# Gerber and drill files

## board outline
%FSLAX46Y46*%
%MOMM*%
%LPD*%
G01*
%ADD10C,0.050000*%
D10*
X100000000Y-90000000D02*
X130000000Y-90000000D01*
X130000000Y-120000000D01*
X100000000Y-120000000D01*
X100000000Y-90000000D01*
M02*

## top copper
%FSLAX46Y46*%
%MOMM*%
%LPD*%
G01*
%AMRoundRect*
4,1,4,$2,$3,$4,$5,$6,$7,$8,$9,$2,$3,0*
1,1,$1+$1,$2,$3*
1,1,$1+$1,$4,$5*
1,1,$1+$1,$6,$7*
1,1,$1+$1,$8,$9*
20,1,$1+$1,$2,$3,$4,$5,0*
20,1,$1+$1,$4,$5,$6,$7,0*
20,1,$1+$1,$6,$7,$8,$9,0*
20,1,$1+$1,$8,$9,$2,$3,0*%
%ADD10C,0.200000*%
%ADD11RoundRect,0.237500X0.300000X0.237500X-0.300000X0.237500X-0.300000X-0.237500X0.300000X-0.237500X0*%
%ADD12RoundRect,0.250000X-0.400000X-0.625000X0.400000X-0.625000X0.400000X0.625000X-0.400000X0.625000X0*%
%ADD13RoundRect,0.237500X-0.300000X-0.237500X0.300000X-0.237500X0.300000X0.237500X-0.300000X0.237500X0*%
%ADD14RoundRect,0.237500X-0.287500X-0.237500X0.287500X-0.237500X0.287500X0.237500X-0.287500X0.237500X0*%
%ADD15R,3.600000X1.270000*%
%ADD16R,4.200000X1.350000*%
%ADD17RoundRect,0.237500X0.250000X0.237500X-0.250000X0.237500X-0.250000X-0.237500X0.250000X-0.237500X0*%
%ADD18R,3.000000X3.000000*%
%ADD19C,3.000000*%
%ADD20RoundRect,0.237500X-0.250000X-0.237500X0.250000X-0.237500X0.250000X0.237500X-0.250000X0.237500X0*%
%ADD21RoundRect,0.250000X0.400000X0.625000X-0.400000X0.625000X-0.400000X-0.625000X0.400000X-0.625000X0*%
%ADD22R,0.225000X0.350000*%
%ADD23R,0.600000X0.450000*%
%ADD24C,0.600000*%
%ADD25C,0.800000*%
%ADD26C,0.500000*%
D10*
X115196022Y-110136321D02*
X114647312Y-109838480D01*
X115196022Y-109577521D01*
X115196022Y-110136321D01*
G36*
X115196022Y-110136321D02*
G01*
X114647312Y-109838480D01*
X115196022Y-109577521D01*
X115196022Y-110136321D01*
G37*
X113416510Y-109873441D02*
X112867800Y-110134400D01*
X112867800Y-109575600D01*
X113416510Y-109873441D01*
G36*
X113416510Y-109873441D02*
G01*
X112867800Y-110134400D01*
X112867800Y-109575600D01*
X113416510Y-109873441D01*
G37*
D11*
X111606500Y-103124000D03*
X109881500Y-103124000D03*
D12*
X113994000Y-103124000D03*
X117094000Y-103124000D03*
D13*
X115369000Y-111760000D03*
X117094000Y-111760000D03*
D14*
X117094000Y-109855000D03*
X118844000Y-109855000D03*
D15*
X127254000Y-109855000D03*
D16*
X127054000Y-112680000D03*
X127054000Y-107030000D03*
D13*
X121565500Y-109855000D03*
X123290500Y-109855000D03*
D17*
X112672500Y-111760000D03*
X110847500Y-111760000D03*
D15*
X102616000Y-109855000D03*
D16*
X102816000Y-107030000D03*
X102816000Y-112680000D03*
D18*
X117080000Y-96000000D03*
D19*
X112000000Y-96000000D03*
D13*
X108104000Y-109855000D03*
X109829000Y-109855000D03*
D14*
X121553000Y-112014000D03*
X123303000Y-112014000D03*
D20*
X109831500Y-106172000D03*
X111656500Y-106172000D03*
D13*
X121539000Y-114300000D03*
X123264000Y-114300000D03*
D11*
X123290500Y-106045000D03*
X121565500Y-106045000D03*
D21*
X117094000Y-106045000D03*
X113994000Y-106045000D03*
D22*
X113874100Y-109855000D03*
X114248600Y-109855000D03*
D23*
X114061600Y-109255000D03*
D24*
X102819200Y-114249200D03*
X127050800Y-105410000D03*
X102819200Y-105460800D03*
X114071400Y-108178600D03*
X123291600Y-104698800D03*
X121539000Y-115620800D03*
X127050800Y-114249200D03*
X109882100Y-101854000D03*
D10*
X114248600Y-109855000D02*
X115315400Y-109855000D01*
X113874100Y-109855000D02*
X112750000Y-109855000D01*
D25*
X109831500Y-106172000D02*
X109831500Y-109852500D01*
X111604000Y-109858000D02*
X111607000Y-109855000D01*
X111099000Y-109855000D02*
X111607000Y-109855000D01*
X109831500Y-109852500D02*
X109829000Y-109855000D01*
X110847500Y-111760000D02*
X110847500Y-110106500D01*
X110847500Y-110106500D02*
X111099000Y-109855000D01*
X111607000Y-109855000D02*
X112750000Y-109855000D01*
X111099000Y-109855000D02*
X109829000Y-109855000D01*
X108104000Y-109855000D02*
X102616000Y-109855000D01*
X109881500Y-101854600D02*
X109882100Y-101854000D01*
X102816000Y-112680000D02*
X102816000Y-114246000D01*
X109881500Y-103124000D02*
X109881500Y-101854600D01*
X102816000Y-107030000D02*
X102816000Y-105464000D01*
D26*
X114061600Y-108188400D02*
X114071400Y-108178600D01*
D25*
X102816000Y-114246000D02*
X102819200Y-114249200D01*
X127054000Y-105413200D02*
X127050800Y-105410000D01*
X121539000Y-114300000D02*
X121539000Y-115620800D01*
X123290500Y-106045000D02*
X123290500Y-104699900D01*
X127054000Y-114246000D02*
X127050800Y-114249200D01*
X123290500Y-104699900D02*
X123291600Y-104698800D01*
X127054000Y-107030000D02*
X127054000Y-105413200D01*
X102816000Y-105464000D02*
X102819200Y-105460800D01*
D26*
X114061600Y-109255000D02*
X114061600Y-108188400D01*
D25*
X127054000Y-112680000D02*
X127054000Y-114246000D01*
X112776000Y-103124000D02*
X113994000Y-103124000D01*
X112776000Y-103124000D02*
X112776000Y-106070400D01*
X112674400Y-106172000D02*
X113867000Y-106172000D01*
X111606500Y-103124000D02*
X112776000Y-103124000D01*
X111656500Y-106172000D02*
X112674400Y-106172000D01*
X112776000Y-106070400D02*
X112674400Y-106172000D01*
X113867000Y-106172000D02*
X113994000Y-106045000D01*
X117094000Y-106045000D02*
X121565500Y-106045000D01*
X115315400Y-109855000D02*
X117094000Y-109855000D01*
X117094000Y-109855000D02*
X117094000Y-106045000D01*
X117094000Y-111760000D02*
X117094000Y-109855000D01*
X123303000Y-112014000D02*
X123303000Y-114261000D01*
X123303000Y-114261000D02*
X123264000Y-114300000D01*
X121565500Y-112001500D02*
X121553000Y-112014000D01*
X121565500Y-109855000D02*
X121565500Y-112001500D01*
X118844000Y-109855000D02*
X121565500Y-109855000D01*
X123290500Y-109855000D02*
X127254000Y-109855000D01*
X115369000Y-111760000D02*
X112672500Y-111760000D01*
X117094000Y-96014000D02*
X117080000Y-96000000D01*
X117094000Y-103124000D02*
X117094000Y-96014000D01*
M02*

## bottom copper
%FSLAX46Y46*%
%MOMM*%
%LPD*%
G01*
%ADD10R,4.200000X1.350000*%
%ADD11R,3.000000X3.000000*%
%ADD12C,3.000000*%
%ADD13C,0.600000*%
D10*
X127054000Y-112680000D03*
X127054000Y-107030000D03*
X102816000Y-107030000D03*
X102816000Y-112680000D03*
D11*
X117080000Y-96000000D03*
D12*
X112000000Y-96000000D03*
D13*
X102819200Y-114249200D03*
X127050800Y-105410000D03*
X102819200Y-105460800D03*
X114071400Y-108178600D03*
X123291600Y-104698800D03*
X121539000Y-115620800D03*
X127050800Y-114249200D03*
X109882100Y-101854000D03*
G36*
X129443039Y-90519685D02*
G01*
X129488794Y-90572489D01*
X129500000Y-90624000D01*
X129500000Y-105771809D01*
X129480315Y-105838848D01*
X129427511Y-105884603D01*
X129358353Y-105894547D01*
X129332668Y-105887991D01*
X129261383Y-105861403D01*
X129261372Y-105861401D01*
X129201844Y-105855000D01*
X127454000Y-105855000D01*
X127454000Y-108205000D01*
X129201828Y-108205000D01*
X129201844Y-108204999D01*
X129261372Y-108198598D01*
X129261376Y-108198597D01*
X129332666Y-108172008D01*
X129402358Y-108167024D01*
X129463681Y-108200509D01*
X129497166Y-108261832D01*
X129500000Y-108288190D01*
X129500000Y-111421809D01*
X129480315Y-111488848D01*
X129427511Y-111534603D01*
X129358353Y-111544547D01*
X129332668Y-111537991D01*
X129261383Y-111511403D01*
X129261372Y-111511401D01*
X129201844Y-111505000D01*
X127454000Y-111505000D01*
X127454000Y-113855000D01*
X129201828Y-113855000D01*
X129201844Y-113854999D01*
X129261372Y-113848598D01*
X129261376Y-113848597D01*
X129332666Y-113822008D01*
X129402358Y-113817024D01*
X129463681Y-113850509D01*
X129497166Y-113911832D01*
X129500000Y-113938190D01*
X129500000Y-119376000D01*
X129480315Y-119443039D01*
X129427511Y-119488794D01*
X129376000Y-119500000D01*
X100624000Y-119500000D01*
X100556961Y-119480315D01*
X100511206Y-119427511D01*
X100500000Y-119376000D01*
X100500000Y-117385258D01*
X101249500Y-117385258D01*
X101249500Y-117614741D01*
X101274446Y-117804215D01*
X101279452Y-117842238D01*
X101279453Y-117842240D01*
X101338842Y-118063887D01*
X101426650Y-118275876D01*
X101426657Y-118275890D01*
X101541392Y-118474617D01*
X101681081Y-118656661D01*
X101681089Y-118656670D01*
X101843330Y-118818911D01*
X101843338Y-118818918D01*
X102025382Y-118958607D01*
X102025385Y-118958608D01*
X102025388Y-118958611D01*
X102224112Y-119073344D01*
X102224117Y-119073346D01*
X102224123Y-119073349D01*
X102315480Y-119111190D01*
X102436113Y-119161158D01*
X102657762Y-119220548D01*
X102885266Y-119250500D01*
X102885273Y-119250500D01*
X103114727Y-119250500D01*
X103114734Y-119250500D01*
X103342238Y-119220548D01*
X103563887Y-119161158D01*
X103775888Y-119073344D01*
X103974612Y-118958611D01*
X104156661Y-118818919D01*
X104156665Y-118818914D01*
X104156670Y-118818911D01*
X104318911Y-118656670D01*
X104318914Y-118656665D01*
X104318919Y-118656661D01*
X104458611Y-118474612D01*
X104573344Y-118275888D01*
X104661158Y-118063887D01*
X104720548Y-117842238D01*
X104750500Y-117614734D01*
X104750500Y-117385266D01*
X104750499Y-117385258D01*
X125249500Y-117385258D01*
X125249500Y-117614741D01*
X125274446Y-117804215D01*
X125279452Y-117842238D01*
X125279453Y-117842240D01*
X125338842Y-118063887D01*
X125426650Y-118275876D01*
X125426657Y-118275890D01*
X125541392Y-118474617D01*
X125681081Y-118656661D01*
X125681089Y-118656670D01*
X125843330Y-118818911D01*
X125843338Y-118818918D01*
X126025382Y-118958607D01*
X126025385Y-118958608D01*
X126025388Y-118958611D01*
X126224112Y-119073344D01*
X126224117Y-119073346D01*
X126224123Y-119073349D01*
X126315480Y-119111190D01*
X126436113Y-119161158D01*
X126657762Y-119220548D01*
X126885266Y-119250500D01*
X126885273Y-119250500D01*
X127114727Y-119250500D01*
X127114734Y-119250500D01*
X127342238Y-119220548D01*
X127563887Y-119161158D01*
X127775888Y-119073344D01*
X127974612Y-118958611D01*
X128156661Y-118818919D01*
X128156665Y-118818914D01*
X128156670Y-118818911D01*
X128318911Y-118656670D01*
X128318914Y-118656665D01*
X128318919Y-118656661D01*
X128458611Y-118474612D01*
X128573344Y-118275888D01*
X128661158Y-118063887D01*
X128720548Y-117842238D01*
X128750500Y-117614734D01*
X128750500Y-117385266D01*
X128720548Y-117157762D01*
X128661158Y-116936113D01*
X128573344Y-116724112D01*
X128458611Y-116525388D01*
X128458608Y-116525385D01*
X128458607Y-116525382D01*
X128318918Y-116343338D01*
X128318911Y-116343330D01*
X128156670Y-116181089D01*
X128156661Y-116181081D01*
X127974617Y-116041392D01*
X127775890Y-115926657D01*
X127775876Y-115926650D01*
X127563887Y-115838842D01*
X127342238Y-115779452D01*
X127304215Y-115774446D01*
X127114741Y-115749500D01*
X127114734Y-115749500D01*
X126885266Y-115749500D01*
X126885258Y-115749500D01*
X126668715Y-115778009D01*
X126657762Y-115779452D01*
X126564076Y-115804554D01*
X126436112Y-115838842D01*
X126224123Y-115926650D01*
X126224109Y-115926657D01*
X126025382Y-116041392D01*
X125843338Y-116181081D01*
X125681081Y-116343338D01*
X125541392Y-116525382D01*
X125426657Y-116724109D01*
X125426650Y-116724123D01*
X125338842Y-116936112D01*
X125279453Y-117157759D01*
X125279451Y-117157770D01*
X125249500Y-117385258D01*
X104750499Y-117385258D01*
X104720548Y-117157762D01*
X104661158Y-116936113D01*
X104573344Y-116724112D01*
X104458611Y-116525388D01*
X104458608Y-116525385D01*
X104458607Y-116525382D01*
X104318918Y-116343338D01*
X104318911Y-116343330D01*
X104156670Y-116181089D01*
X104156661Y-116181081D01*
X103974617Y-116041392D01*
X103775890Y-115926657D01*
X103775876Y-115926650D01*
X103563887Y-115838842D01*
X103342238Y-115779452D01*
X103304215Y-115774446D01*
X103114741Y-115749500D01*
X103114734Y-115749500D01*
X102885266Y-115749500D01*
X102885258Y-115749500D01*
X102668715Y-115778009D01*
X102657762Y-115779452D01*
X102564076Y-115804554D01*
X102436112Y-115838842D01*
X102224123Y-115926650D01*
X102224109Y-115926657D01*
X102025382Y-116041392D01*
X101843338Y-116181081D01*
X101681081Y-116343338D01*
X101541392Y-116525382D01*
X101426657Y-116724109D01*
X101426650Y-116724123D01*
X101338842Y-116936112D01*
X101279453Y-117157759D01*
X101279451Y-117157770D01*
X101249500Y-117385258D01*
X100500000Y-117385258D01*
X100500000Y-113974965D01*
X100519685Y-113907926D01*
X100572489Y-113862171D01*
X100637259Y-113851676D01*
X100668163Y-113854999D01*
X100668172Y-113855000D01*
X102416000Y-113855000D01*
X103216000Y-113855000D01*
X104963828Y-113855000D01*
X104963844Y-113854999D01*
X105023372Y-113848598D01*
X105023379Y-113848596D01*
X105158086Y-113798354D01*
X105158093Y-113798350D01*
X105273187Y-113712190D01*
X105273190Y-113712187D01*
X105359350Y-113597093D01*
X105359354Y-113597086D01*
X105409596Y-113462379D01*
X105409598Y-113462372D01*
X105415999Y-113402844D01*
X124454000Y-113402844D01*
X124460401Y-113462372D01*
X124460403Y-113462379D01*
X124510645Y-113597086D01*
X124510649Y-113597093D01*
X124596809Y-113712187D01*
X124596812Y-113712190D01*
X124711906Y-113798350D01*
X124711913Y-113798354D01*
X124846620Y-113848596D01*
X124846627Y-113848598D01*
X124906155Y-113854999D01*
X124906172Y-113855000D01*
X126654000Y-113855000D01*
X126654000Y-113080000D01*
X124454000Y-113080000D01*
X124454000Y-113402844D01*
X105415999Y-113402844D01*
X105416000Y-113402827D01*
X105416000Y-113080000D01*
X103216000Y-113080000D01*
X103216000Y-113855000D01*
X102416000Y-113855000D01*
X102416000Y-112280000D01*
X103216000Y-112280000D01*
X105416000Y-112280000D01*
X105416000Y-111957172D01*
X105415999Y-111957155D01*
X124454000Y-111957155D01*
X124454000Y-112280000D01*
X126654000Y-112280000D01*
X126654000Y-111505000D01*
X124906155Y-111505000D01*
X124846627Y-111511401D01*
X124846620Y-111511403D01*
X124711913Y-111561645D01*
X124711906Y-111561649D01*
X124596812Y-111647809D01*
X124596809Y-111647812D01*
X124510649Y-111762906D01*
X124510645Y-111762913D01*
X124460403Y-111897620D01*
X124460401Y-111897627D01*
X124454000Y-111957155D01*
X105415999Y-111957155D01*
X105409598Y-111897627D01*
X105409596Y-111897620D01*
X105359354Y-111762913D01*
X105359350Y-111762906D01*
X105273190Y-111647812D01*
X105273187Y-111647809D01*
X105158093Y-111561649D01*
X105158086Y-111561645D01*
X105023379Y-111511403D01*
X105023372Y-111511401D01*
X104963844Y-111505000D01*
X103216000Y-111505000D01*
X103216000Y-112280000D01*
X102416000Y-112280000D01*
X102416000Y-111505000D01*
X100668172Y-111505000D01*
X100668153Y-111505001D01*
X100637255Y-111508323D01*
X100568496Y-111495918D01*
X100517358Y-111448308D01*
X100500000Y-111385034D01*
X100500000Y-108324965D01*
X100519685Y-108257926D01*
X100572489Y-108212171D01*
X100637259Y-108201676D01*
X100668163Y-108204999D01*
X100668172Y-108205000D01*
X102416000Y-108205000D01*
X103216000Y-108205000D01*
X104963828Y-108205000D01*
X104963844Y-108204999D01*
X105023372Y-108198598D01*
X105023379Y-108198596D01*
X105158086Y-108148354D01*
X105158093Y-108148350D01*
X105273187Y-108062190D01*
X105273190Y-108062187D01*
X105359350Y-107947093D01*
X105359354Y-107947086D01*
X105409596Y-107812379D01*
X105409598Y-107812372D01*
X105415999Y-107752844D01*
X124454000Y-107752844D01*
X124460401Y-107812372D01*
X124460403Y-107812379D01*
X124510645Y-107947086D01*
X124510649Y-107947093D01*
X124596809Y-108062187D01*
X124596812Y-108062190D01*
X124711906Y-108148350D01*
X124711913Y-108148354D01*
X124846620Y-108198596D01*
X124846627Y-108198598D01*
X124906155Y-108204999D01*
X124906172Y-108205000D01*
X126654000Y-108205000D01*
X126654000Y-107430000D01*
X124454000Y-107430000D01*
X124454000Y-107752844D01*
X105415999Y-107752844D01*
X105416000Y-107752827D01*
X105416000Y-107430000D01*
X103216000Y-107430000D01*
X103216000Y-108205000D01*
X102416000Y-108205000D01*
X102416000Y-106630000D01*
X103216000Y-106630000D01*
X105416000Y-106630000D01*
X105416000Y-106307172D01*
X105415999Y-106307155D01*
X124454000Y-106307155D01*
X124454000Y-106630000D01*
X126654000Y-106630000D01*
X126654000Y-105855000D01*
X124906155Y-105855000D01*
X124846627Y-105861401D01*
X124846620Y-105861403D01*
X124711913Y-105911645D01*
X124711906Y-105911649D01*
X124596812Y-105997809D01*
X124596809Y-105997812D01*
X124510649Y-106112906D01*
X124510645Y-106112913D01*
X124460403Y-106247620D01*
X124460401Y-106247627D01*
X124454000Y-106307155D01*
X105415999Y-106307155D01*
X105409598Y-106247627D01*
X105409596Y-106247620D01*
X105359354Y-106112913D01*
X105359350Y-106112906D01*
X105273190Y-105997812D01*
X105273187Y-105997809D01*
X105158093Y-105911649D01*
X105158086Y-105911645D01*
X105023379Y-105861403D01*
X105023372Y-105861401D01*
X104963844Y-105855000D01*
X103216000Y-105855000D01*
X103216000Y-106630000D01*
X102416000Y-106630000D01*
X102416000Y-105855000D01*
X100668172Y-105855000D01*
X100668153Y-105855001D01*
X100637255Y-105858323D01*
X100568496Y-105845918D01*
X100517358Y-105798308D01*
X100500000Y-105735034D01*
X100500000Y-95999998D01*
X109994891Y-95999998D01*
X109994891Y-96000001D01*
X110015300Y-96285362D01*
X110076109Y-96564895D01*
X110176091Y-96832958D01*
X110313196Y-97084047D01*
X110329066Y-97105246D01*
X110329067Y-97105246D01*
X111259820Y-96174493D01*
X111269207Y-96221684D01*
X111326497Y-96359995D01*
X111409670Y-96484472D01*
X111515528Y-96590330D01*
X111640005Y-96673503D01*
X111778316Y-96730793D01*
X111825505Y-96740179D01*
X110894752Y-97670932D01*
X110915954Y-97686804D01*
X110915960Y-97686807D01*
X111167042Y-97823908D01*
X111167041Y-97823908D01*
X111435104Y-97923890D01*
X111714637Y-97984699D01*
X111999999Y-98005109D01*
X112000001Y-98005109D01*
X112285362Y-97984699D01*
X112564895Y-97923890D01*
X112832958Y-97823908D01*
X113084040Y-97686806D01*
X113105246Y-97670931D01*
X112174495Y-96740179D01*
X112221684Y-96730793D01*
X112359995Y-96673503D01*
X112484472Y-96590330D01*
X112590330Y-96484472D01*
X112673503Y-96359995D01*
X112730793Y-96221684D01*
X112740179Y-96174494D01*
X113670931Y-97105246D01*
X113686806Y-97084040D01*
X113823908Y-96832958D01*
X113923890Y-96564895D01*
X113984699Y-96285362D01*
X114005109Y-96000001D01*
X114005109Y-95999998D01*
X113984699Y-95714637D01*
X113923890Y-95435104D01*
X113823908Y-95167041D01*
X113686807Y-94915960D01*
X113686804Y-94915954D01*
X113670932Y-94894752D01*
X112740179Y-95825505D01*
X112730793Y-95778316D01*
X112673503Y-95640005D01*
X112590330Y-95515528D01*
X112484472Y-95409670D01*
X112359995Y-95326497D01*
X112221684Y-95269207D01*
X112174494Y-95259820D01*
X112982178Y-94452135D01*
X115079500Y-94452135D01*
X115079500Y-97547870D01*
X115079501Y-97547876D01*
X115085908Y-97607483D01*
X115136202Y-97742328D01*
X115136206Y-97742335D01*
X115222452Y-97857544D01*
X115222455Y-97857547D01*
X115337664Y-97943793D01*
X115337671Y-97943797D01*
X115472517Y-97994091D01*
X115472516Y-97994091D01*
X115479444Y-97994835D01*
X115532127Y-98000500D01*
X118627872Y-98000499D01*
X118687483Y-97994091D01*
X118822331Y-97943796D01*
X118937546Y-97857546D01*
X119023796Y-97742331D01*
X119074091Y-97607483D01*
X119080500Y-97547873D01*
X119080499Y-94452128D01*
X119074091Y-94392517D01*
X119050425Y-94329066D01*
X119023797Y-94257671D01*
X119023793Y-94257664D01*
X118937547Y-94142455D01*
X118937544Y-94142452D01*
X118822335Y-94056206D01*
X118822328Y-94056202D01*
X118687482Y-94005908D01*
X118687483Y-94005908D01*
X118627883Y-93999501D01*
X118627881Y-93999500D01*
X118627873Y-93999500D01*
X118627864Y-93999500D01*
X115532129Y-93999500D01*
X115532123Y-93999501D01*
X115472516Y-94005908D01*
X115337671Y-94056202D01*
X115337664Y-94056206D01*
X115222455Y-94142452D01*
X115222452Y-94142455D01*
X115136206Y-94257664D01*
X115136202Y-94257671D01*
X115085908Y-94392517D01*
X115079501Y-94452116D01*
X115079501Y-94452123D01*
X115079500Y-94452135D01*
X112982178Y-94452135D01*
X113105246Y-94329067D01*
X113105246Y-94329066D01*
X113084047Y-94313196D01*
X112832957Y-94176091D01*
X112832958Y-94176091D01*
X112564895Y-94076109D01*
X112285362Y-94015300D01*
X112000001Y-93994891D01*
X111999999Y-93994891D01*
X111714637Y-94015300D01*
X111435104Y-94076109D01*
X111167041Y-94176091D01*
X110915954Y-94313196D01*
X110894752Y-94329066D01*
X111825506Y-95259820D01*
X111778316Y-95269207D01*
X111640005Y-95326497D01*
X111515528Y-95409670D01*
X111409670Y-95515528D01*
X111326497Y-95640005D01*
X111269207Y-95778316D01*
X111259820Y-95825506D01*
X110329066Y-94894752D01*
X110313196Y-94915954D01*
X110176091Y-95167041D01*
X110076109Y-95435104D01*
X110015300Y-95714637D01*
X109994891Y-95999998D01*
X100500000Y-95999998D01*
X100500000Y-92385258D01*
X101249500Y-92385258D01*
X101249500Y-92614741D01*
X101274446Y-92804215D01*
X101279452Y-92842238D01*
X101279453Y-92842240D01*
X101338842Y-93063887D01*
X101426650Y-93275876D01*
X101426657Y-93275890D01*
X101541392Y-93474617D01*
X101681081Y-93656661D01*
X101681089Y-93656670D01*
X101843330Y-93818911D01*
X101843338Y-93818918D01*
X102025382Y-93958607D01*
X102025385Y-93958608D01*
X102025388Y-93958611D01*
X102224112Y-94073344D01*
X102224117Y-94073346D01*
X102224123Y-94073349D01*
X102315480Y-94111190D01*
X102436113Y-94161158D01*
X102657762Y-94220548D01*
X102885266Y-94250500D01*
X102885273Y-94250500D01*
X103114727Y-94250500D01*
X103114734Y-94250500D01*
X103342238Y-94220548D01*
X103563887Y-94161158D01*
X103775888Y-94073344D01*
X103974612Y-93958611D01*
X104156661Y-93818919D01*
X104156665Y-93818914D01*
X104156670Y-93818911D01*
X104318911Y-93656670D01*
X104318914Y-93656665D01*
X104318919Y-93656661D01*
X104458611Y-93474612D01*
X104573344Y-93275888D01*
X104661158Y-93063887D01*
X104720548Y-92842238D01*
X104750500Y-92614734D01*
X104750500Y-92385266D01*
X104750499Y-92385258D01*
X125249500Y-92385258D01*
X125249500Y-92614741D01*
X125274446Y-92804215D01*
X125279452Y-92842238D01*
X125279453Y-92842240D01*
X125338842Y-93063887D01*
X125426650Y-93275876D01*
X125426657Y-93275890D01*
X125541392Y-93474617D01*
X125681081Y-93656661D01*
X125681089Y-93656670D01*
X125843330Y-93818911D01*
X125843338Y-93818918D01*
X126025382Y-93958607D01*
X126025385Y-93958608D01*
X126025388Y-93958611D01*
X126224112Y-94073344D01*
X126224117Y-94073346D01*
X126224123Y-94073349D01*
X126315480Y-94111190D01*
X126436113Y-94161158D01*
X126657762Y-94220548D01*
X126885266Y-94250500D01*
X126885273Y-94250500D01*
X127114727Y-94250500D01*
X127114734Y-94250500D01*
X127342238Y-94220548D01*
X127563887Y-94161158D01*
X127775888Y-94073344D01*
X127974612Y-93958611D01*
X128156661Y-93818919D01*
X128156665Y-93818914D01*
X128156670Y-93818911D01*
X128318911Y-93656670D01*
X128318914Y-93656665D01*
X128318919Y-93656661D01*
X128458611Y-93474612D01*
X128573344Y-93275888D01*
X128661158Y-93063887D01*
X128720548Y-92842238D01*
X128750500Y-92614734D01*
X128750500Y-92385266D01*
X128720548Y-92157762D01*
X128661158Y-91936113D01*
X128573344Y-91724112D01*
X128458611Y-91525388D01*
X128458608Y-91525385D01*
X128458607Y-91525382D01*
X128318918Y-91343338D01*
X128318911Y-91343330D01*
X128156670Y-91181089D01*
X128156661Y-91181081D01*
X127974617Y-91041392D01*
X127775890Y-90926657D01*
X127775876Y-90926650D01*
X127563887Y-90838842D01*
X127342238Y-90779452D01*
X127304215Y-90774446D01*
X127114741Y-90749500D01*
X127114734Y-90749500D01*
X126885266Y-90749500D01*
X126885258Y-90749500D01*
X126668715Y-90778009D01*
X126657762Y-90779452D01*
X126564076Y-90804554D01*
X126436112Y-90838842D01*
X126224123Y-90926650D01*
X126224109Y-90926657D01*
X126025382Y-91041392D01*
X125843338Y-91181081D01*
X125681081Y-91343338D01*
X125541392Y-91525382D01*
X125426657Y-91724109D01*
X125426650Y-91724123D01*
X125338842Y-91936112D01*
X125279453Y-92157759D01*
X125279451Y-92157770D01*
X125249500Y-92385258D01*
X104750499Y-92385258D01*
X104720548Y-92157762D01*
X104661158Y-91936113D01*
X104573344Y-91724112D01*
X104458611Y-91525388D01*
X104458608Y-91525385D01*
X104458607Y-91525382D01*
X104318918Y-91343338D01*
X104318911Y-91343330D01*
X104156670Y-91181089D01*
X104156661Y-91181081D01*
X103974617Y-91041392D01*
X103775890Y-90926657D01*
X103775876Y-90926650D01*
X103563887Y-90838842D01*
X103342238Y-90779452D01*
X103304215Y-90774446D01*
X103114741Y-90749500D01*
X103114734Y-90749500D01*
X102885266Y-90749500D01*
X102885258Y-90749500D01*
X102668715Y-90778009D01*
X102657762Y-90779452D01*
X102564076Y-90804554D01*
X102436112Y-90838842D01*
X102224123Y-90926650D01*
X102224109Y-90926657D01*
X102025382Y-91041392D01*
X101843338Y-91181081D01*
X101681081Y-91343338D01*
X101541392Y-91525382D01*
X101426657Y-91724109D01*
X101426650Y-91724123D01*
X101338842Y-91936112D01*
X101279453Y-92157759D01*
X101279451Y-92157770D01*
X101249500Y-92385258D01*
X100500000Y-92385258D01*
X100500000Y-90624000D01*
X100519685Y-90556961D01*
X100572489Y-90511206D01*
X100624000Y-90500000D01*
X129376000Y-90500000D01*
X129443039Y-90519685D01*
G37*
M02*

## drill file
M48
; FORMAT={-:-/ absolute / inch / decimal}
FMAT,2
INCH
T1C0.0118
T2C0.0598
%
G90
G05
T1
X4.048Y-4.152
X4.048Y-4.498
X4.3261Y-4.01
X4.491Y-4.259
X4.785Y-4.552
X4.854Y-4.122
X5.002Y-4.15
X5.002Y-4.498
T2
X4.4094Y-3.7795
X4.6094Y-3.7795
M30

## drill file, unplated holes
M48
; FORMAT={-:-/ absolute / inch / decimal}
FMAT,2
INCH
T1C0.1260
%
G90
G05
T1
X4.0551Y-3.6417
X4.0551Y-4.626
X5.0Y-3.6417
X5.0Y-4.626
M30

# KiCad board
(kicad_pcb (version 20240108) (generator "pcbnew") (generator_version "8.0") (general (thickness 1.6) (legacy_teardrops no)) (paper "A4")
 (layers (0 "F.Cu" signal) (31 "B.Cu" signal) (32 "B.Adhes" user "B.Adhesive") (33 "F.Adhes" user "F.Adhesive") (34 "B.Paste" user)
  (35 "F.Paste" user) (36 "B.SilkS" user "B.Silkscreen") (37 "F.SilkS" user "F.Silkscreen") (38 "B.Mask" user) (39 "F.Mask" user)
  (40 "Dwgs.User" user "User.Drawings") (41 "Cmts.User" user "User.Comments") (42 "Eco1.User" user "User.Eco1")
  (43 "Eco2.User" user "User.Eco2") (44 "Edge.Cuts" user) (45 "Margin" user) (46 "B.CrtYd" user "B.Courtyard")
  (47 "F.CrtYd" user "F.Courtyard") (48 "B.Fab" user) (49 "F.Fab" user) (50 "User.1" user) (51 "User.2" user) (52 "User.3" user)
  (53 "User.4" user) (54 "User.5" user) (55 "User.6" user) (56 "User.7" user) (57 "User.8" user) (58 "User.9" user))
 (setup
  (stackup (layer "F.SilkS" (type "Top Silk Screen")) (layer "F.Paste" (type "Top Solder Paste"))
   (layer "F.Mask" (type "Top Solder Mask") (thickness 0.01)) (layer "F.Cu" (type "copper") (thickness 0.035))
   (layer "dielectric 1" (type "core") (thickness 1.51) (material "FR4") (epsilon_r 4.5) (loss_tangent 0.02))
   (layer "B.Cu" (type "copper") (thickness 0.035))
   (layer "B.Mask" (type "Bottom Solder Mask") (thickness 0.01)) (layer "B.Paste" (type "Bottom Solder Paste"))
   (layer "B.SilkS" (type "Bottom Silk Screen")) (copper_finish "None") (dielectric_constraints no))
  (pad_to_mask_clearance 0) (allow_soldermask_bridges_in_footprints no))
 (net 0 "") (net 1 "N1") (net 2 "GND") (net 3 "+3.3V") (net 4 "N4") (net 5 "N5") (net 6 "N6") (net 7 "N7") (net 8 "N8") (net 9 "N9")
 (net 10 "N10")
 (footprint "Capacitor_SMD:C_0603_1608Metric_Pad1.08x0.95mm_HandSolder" (layer "F.Cu") (at 110.744 103.124 180)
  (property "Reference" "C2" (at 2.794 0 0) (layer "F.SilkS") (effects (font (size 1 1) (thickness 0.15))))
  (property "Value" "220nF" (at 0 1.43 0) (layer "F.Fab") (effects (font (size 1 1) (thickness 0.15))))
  (pad "1" smd roundrect (at -0.8625 0 180) (size 1.075 0.95) (layers "F.Cu" "F.Paste" "F.Mask") (roundrect_rratio 0.25) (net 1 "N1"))
  (pad "2" smd roundrect (at 0.8625 0 180) (size 1.075 0.95) (layers "F.Cu" "F.Paste" "F.Mask") (roundrect_rratio 0.25) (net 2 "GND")))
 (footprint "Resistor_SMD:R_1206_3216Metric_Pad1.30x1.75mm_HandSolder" (layer "F.Cu") (at 115.544 103.124)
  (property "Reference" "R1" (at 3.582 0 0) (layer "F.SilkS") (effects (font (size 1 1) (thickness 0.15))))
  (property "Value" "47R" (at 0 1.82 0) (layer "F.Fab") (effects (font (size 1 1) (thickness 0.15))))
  (pad "1" smd roundrect (at -1.55 0) (size 1.3 1.75) (layers "F.Cu" "F.Paste" "F.Mask") (roundrect_rratio 0.192308) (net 1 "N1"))
  (pad "2" smd roundrect (at 1.55 0) (size 1.3 1.75) (layers "F.Cu" "F.Paste" "F.Mask") (roundrect_rratio 0.192308) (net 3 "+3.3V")))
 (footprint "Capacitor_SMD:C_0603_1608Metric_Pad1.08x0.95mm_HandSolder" (layer "F.Cu") (at 116.2315 111.76)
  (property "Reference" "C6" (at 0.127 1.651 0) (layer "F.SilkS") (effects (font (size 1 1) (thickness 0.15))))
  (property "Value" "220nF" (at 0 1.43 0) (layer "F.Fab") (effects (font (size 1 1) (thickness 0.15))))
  (pad "1" smd roundrect (at -0.8625 0) (size 1.075 0.95) (layers "F.Cu" "F.Paste" "F.Mask") (roundrect_rratio 0.25) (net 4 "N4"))
  (pad "2" smd roundrect (at 0.8625 0) (size 1.075 0.95) (layers "F.Cu" "F.Paste" "F.Mask") (roundrect_rratio 0.25) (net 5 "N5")))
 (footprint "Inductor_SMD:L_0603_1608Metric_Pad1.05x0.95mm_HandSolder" (layer "F.Cu") (at 117.969 109.855)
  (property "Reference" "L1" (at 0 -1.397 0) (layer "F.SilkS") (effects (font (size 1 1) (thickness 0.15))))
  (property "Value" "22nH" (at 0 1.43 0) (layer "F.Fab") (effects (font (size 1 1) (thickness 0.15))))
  (pad "1" smd roundrect (at -0.875 0) (size 1.05 0.95) (layers "F.Cu" "F.Paste" "F.Mask") (roundrect_rratio 0.25) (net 5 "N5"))
  (pad "2" smd roundrect (at 0.875 0) (size 1.05 0.95) (layers "F.Cu" "F.Paste" "F.Mask") (roundrect_rratio 0.25) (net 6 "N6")))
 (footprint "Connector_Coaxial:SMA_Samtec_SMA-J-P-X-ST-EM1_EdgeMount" (layer "F.Cu") (at 127.054 109.855 90)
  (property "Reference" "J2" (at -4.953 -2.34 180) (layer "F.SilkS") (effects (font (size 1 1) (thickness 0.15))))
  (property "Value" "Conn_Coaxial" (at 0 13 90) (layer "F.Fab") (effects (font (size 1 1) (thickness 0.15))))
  (pad "1" smd rect (at 0 0.2 90) (size 1.27 3.6) (layers "F.Cu" "F.Paste" "F.Mask") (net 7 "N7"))
  (pad "2" smd rect (at -2.825 0 90) (size 1.35 4.2) (layers "F.Cu" "F.Paste" "F.Mask") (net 2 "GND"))
  (pad "2" smd rect (at -2.825 0 90) (size 1.35 4.2) (layers "B.Cu" "B.Paste" "B.Mask") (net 2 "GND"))
  (pad "2" smd rect (at 2.825 0 90) (size 1.35 4.2) (layers "F.Cu" "F.Paste" "F.Mask") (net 2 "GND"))
  (pad "2" smd rect (at 2.825 0 90) (size 1.35 4.2) (layers "B.Cu" "B.Paste" "B.Mask") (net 2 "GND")))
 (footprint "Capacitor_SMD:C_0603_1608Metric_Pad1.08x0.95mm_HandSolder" (layer "F.Cu") (at 122.428 109.855)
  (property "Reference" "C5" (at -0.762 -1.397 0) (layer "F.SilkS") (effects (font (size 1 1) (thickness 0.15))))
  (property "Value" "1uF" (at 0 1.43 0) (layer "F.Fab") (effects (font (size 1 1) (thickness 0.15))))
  (pad "1" smd roundrect (at -0.8625 0) (size 1.075 0.95) (layers "F.Cu" "F.Paste" "F.Mask") (roundrect_rratio 0.25) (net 6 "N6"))
  (pad "2" smd roundrect (at 0.8625 0) (size 1.075 0.95) (layers "F.Cu" "F.Paste" "F.Mask") (roundrect_rratio 0.25) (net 7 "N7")))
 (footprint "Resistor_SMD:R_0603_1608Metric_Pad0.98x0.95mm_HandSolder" (layer "F.Cu") (at 111.76 111.76 180)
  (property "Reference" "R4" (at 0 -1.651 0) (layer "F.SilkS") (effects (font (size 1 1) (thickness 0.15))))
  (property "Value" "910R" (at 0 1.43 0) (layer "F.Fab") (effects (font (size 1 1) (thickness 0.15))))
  (pad "1" smd roundrect (at -0.9125 0 180) (size 0.975 0.95) (layers "F.Cu" "F.Paste" "F.Mask") (roundrect_rratio 0.25) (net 4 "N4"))
  (pad "2" smd roundrect (at 0.9125 0 180) (size 0.975 0.95) (layers "F.Cu" "F.Paste" "F.Mask") (roundrect_rratio 0.25) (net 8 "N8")))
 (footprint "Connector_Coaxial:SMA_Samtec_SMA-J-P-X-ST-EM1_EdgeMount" (layer "F.Cu") (at 102.816 109.855 -90)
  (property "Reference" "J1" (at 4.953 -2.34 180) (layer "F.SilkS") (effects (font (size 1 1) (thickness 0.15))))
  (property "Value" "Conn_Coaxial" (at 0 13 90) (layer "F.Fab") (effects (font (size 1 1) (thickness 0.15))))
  (pad "1" smd rect (at 0 0.2 270) (size 1.27 3.6) (layers "F.Cu" "F.Paste" "F.Mask") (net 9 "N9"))
  (pad "2" smd rect (at -2.825 0 270) (size 1.35 4.2) (layers "F.Cu" "F.Paste" "F.Mask") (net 2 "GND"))
  (pad "2" smd rect (at -2.825 0 270) (size 1.35 4.2) (layers "B.Cu" "B.Paste" "B.Mask") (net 2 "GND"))
  (pad "2" smd rect (at 2.825 0 270) (size 1.35 4.2) (layers "F.Cu" "F.Paste" "F.Mask") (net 2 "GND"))
  (pad "2" smd rect (at 2.825 0 270) (size 1.35 4.2) (layers "B.Cu" "B.Paste" "B.Mask") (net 2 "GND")))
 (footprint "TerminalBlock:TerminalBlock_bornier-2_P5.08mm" (layer "F.Cu") (at 117.08 96 180)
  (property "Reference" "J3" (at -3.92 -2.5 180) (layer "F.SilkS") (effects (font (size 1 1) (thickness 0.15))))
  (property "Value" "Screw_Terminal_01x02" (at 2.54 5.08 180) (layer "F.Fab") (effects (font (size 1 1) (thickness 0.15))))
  (pad "1" thru_hole rect (at 0 0 180) (size 3 3) (drill 1.52) (layers "*.Cu" "*.Mask") (remove_unused_layers no) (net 3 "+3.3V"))
  (pad "2" thru_hole circle (at 5.08 0 180) (size 3 3) (drill 1.52) (layers "*.Cu" "*.Mask") (remove_unused_layers no) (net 2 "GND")))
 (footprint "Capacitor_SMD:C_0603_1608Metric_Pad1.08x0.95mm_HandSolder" (layer "F.Cu") (at 108.9665 109.855)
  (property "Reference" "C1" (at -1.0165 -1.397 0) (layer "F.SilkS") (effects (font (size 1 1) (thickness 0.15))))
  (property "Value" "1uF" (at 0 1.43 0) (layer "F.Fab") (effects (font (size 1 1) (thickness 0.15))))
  (pad "1" smd roundrect (at -0.8625 0) (size 1.075 0.95) (layers "F.Cu" "F.Paste" "F.Mask") (roundrect_rratio 0.25) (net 9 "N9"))
  (pad "2" smd roundrect (at 0.8625 0) (size 1.075 0.95) (layers "F.Cu" "F.Paste" "F.Mask") (roundrect_rratio 0.25) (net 8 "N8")))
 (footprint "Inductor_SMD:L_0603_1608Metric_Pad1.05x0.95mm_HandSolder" (layer "F.Cu") (at 122.428 112.014)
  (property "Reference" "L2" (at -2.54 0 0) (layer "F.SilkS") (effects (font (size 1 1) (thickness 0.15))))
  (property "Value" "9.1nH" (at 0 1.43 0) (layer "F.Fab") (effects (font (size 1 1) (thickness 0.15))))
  (pad "1" smd roundrect (at -0.875 0) (size 1.05 0.95) (layers "F.Cu" "F.Paste" "F.Mask") (roundrect_rratio 0.25) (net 6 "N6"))
  (pad "2" smd roundrect (at 0.875 0) (size 1.05 0.95) (layers "F.Cu" "F.Paste" "F.Mask") (roundrect_rratio 0.25) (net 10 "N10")))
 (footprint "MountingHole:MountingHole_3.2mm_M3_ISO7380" (layer "F.Cu") (at 103 92.5)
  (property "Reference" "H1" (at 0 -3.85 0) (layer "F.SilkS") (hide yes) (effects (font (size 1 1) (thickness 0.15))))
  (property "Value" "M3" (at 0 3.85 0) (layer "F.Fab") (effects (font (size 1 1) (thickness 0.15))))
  (pad "" np_thru_hole circle (at 0 0) (size 3.2 3.2) (drill 3.2) (layers "*.Cu" "*.Mask")))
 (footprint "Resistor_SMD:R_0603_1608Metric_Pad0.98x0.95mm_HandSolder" (layer "F.Cu") (at 110.744 106.172)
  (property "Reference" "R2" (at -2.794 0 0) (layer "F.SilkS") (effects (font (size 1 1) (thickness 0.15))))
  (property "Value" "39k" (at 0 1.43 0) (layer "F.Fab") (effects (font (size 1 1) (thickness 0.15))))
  (pad "1" smd roundrect (at -0.9125 0) (size 0.975 0.95) (layers "F.Cu" "F.Paste" "F.Mask") (roundrect_rratio 0.25) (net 8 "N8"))
  (pad "2" smd roundrect (at 0.9125 0) (size 0.975 0.95) (layers "F.Cu" "F.Paste" "F.Mask") (roundrect_rratio 0.25) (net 1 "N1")))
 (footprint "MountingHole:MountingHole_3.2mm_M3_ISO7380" (layer "F.Cu") (at 127 92.5)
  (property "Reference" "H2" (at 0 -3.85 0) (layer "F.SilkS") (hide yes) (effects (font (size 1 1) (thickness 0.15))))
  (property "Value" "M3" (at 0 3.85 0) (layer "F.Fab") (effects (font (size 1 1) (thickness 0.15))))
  (pad "" np_thru_hole circle (at 0 0) (size 3.2 3.2) (drill 3.2) (layers "*.Cu" "*.Mask")))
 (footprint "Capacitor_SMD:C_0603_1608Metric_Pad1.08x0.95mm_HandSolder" (layer "F.Cu") (at 122.4015 114.3)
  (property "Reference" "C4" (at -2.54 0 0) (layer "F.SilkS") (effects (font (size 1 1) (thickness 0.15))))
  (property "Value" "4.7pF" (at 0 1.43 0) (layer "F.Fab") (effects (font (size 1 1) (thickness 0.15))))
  (pad "1" smd roundrect (at -0.8625 0) (size 1.075 0.95) (layers "F.Cu" "F.Paste" "F.Mask") (roundrect_rratio 0.25) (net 2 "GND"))
  (pad "2" smd roundrect (at 0.8625 0) (size 1.075 0.95) (layers "F.Cu" "F.Paste" "F.Mask") (roundrect_rratio 0.25) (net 10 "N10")))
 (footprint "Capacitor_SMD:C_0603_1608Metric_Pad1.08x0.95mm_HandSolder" (layer "F.Cu") (at 122.428 106.045 180)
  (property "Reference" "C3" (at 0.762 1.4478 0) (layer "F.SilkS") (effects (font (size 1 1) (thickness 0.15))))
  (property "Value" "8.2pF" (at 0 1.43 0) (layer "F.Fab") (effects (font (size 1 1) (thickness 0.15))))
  (pad "1" smd roundrect (at -0.8625 0 180) (size 1.075 0.95) (layers "F.Cu" "F.Paste" "F.Mask") (roundrect_rratio 0.25) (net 2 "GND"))
  (pad "2" smd roundrect (at 0.8625 0 180) (size 1.075 0.95) (layers "F.Cu" "F.Paste" "F.Mask") (roundrect_rratio 0.25) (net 5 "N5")))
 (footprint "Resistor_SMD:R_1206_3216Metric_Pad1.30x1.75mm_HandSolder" (layer "F.Cu") (at 115.544 106.045 180)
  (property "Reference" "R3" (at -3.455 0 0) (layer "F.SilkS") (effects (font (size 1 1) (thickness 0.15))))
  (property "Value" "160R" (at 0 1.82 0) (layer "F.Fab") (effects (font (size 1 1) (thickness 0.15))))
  (pad "1" smd roundrect (at -1.55 0 180) (size 1.3 1.75) (layers "F.Cu" "F.Paste" "F.Mask") (roundrect_rratio 0.192308) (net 5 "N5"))
  (pad "2" smd roundrect (at 1.55 0 180) (size 1.3 1.75) (layers "F.Cu" "F.Paste" "F.Mask") (roundrect_rratio 0.192308) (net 1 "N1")))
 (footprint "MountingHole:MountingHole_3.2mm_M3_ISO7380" (layer "F.Cu") (at 127 117.5)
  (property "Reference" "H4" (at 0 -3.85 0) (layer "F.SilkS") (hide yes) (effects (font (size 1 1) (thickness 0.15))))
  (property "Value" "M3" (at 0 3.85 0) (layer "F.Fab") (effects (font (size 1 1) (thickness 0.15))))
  (pad "" np_thru_hole circle (at 0 0) (size 3.2 3.2) (drill 3.2) (layers "*.Cu" "*.Mask")))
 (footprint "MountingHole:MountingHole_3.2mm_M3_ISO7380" (layer "F.Cu") (at 103 117.5)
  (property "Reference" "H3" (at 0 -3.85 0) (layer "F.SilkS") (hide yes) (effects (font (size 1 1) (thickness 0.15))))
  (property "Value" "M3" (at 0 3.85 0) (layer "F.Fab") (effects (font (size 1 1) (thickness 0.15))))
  (pad "" np_thru_hole circle (at 0 0) (size 3.2 3.2) (drill 3.2) (layers "*.Cu" "*.Mask")))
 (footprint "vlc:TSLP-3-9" (layer "F.Cu") (at 114.06135 109.555 90)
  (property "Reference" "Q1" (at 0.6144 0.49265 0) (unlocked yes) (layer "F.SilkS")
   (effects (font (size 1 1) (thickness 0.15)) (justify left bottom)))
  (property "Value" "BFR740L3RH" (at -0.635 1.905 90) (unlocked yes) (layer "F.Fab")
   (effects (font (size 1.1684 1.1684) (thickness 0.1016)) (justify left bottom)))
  (pad "1" smd rect (at -0.3 -0.18725 90) (size 0.35 0.225) (layers "F.Cu" "F.Paste") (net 8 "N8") (solder_mask_margin 0.1016)
   (clearance 0.15) (thermal_bridge_angle 0))
  (pad "2" smd rect (at -0.3 0.18725 90) (size 0.35 0.225) (layers "F.Cu" "F.Paste") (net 5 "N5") (solder_mask_margin 0.1016)
   (clearance 0.15) (thermal_bridge_angle 0))
  (pad "3" smd rect (at 0.3 0.00025 90) (size 0.45 0.6) (layers "F.Cu" "F.Paste") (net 2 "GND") (solder_mask_margin 0.1016)
   (thermal_bridge_angle 0)))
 (gr_poly
  (pts (xy 115.196022 109.577521) (xy 114.647312 109.83848) (xy 115.196022 110.136321)) (stroke (width 0.2) (type solid)) (fill solid)
  (layer "F.Cu") (net 5))
 (gr_poly
  (pts (xy 112.8678 110.1344) (xy 113.41651 109.873441) (xy 112.8678 109.5756)) (stroke (width 0.2) (type solid)) (fill solid)
  (layer "F.Cu") (net 8))
 (gr_rect (start 100 90) (end 130 120) (stroke (width 0.05) (type default)) (fill none) (layer "Edge.Cuts"))
 (segment (start 109.8315 106.172) (end 109.8315 109.8525) (width 0.8) (layer "F.Cu") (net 8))
 (segment (start 111.604 109.858) (end 111.607 109.855) (width 0.8) (layer "F.Cu") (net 8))
 (segment (start 111.099 109.855) (end 111.607 109.855) (width 0.8) (layer "F.Cu") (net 8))
 (segment (start 109.8315 109.8525) (end 109.829 109.855) (width 0.8) (layer "F.Cu") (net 8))
 (segment (start 110.8475 111.76) (end 110.8475 110.1065) (width 0.8) (layer "F.Cu") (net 8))
 (segment (start 110.8475 110.1065) (end 111.099 109.855) (width 0.8) (layer "F.Cu") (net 8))
 (segment (start 111.607 109.855) (end 112.75 109.855) (width 0.8) (layer "F.Cu") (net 8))
 (segment (start 113.8741 109.855) (end 112.75 109.855) (width 0.2) (layer "F.Cu") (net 8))
 (segment (start 111.099 109.855) (end 109.829 109.855) (width 0.8) (layer "F.Cu") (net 8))
 (segment (start 108.104 109.855) (end 102.616 109.855) (width 0.8) (layer "F.Cu") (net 9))
 (segment (start 109.8815 101.8546) (end 109.8821 101.854) (width 0.8) (layer "F.Cu") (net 2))
 (segment (start 102.816 112.68) (end 102.816 114.246) (width 0.8) (layer "F.Cu") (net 2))
 (segment (start 109.8815 103.124) (end 109.8815 101.8546) (width 0.8) (layer "F.Cu") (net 2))
 (segment (start 102.816 107.03) (end 102.816 105.464) (width 0.8) (layer "F.Cu") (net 2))
 (segment (start 114.0616 108.1884) (end 114.0714 108.1786) (width 0.5) (layer "F.Cu") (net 2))
 (segment (start 102.816 114.246) (end 102.8192 114.2492) (width 0.8) (layer "F.Cu") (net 2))
 (segment (start 127.054 105.4132) (end 127.0508 105.41) (width 0.8) (layer "F.Cu") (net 2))
 (segment (start 121.539 114.3) (end 121.539 115.6208) (width 0.8) (layer "F.Cu") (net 2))
 (segment (start 123.2905 106.045) (end 123.2905 104.6999) (width 0.8) (layer "F.Cu") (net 2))
 (segment (start 127.054 114.246) (end 127.0508 114.2492) (width 0.8) (layer "F.Cu") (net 2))
 (segment (start 123.2905 104.6999) (end 123.2916 104.6988) (width 0.8) (layer "F.Cu") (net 2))
 (segment (start 127.054 107.03) (end 127.054 105.4132) (width 0.8) (layer "F.Cu") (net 2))
 (segment (start 102.816 105.464) (end 102.8192 105.4608) (width 0.8) (layer "F.Cu") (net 2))
 (segment (start 114.0616 109.255) (end 114.0616 108.1884) (width 0.5) (layer "F.Cu") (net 2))
 (segment (start 127.054 112.68) (end 127.054 114.246) (width 0.8) (layer "F.Cu") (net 2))
 (via (at 102.8192 114.2492) (size 0.6) (drill 0.3) (layers "F.Cu" "B.Cu") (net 2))
 (via (at 127.0508 105.41) (size 0.6) (drill 0.3) (layers "F.Cu" "B.Cu") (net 2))
 (via (at 102.8192 105.4608) (size 0.6) (drill 0.3) (layers "F.Cu" "B.Cu") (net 2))
 (via (at 114.0714 108.1786) (size 0.6) (drill 0.3) (layers "F.Cu" "B.Cu") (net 2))
 (via (at 123.2916 104.6988) (size 0.6) (drill 0.3) (layers "F.Cu" "B.Cu") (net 2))
 (via (at 121.539 115.6208) (size 0.6) (drill 0.3) (layers "F.Cu" "B.Cu") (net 2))
 (via (at 127.0508 114.2492) (size 0.6) (drill 0.3) (layers "F.Cu" "B.Cu") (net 2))
 (via (at 109.8821 101.854) (size 0.6) (drill 0.3) (layers "F.Cu" "B.Cu") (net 2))
 (segment (start 112.776 103.124) (end 113.994 103.124) (width 0.8) (layer "F.Cu") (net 1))
 (segment (start 112.776 103.124) (end 112.776 106.0704) (width 0.8) (layer "F.Cu") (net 1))
 (segment (start 112.6744 106.172) (end 113.867 106.172) (width 0.8) (layer "F.Cu") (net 1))
 (segment (start 111.6065 103.124) (end 112.776 103.124) (width 0.8) (layer "F.Cu") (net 1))
 (segment (start 111.6565 106.172) (end 112.6744 106.172) (width 0.8) (layer "F.Cu") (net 1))
 (segment (start 112.776 106.0704) (end 112.6744 106.172) (width 0.8) (layer "F.Cu") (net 1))
 (segment (start 113.867 106.172) (end 113.994 106.045) (width 0.8) (layer "F.Cu") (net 1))
 (segment (start 117.094 106.045) (end 121.5655 106.045) (width 0.8) (layer "F.Cu") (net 5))
 (segment (start 115.3154 109.855) (end 117.094 109.855) (width 0.8) (layer "F.Cu") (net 5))
 (segment (start 117.094 109.855) (end 117.094 106.045) (width 0.8) (layer "F.Cu") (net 5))
 (segment (start 117.094 111.76) (end 117.094 109.855) (width 0.8) (layer "F.Cu") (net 5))
 (segment (start 114.2486 109.855) (end 115.3154 109.855) (width 0.2) (layer "F.Cu") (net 5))
 (segment (start 123.303 112.014) (end 123.303 114.261) (width 0.8) (layer "F.Cu") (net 10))
 (segment (start 123.303 114.261) (end 123.264 114.3) (width 0.8) (layer "F.Cu") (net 10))
 (segment (start 121.5655 112.0015) (end 121.553 112.014) (width 0.8) (layer "F.Cu") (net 6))
 (segment (start 121.5655 109.855) (end 121.5655 112.0015) (width 0.8) (layer "F.Cu") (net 6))
 (segment (start 118.844 109.855) (end 121.5655 109.855) (width 0.8) (layer "F.Cu") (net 6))
 (segment (start 123.2905 109.855) (end 127.254 109.855) (width 0.8) (layer "F.Cu") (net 7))
 (segment (start 115.369 111.76) (end 112.6725 111.76) (width 0.8) (layer "F.Cu") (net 4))
 (segment (start 117.094 96.014) (end 117.08 96) (width 0.8) (layer "F.Cu") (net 3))
 (segment (start 117.094 103.124) (end 117.094 96.014) (width 0.8) (layer "F.Cu") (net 3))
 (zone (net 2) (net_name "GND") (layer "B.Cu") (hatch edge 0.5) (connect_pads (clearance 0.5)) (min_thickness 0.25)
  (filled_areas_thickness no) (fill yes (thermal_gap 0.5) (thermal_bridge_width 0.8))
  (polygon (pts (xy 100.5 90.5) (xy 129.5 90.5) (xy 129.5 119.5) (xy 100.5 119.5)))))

